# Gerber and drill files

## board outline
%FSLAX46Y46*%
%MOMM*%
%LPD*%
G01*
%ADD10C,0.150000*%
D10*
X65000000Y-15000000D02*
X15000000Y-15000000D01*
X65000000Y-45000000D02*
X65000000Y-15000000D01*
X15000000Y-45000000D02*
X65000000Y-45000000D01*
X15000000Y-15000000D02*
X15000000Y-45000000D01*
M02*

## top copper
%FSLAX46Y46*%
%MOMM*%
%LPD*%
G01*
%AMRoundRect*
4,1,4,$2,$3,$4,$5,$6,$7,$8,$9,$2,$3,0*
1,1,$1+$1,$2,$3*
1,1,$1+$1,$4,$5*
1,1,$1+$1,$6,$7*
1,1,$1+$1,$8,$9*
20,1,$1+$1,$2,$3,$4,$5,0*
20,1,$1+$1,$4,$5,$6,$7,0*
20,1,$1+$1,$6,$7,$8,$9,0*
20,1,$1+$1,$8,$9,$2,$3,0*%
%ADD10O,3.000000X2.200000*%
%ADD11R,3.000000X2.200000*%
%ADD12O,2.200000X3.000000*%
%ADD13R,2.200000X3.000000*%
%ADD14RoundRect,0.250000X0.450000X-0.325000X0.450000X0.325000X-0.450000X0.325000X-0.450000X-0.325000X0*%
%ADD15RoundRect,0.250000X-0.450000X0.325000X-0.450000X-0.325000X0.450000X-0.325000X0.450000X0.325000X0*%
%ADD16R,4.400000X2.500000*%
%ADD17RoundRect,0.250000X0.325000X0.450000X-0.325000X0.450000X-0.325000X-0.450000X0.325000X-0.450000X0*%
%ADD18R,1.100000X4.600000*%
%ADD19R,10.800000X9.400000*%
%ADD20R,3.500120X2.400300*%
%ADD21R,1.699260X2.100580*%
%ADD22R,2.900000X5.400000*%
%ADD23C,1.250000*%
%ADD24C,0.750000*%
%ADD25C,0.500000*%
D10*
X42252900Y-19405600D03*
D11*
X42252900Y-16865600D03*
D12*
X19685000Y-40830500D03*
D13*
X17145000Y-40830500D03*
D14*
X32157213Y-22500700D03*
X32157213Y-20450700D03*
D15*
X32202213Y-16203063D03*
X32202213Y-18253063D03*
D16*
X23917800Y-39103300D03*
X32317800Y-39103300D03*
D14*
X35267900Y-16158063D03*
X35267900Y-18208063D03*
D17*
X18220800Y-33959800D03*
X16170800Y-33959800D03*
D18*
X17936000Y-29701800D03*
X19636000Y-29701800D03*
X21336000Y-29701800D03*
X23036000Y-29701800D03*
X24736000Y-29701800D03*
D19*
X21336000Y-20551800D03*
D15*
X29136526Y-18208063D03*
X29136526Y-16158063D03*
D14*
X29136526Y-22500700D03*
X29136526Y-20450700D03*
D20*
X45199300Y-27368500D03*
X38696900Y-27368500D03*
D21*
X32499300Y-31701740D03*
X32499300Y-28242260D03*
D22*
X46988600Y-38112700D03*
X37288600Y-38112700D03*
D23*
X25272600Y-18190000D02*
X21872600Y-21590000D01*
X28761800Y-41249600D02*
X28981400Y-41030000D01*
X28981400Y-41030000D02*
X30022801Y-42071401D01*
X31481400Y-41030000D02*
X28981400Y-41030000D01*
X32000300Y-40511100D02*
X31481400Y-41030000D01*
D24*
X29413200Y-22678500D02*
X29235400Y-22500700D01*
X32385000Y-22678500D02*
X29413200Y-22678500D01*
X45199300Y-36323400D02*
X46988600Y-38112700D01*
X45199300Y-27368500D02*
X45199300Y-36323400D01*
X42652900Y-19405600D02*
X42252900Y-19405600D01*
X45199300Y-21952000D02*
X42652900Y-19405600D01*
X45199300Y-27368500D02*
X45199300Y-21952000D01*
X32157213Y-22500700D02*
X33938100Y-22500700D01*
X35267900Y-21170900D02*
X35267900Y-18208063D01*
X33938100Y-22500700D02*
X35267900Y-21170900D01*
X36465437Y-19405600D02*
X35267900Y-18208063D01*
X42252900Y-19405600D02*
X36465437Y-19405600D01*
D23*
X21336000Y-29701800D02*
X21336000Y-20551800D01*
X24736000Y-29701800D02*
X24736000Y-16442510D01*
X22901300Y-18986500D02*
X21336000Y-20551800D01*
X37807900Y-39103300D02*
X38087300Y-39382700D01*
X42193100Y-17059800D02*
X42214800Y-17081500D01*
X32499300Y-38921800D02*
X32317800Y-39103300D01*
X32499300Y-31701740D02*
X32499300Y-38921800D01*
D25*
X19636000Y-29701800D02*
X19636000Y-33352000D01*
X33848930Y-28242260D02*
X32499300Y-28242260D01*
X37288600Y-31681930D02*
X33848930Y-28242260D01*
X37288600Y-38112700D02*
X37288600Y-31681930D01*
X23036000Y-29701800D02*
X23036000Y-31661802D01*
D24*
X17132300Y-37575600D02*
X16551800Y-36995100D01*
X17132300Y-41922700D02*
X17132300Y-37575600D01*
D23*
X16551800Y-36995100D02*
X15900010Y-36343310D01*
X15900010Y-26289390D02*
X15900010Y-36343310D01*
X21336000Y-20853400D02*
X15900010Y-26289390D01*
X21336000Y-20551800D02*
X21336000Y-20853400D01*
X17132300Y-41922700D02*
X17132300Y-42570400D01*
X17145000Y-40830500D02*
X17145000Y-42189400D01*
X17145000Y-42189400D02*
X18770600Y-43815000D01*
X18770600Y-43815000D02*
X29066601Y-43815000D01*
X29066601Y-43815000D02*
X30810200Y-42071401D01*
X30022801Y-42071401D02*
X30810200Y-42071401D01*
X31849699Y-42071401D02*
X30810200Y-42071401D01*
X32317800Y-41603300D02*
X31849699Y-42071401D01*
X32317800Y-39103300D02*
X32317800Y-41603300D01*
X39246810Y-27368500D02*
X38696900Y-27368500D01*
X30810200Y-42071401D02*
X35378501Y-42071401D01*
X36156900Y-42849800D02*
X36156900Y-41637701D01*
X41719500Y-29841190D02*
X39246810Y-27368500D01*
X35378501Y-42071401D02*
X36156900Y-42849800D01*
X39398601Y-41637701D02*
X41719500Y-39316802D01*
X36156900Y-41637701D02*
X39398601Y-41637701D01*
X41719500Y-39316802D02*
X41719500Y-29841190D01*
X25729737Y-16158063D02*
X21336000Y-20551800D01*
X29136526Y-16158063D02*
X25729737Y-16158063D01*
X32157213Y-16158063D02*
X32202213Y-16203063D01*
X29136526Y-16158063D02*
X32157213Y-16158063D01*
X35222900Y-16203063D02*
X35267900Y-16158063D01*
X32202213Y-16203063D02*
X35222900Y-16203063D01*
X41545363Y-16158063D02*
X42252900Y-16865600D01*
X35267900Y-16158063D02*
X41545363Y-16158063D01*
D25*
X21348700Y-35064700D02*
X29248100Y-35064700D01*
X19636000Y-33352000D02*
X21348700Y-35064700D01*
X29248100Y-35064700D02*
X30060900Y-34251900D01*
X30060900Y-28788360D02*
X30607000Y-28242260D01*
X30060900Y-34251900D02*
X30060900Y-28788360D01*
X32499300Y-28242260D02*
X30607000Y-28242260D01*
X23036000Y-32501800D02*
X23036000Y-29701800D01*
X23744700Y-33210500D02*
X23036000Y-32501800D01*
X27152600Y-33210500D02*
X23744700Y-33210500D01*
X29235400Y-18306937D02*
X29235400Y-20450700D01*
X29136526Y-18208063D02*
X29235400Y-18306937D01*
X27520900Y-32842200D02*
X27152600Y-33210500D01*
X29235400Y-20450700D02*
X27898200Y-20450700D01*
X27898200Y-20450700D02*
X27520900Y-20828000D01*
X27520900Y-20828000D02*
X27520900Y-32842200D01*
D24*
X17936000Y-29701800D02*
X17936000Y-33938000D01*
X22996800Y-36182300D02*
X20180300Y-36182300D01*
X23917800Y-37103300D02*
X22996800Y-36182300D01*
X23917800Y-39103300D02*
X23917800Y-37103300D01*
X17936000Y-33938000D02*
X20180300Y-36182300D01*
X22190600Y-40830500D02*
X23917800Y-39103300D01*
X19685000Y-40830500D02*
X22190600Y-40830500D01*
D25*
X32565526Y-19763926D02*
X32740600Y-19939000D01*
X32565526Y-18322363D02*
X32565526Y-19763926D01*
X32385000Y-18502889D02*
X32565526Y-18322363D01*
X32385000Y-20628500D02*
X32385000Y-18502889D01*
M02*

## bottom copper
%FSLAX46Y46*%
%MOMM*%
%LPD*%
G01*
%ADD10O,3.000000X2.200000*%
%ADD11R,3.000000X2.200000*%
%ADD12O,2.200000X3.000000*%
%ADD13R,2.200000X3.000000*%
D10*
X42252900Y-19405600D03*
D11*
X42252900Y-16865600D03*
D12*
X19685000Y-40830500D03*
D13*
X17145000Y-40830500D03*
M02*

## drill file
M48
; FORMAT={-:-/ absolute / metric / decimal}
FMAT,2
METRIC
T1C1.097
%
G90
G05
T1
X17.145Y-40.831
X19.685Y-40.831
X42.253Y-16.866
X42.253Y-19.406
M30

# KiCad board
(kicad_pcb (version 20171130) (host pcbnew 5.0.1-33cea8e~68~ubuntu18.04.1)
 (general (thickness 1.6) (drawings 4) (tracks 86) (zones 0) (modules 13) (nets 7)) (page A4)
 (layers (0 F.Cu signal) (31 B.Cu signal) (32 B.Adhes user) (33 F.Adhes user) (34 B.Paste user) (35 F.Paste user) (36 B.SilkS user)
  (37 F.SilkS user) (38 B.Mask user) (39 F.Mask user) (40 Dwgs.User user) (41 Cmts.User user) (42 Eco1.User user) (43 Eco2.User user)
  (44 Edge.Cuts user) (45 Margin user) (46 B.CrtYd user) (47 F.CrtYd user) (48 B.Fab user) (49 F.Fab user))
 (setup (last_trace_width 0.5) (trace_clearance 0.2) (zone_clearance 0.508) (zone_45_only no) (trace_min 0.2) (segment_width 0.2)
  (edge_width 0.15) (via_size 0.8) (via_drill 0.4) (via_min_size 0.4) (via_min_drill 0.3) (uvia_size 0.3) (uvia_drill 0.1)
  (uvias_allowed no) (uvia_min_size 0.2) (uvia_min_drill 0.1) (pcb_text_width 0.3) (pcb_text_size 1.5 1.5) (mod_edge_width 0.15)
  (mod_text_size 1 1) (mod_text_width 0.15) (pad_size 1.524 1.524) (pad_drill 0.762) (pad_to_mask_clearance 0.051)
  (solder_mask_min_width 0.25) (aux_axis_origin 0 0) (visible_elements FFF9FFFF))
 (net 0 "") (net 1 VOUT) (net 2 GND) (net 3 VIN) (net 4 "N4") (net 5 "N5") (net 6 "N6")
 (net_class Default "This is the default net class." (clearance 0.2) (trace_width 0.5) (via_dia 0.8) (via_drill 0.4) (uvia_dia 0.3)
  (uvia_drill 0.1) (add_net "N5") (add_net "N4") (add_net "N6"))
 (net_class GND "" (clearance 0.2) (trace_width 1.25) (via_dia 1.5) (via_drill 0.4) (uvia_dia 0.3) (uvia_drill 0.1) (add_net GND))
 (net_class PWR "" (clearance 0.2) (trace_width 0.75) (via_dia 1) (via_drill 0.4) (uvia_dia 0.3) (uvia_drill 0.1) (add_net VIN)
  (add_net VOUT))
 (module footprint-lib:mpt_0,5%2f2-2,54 (layer F.Cu) (at 42.2529 18.1356 90)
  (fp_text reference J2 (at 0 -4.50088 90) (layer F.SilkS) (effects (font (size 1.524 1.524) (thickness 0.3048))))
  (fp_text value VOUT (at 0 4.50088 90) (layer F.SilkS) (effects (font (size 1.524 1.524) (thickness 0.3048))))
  (pad 2 thru_hole oval (at -1.27 0 90) (size 2.2 3) (drill 1.09728) (layers *.Cu *.Mask) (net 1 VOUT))
  (pad 1 thru_hole rect (at 1.27 0 90) (size 2.2 3) (drill 1.09728) (layers *.Cu *.Mask) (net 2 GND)))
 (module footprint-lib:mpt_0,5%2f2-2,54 (layer F.Cu) (at 18.415 40.8305 180)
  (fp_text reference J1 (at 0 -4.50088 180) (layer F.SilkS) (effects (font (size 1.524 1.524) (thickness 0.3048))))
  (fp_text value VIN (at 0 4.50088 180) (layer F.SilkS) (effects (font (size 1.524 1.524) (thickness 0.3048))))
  (pad 2 thru_hole oval (at -1.27 0 180) (size 2.2 3) (drill 1.09728) (layers *.Cu *.Mask) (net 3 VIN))
  (pad 1 thru_hole rect (at 1.27 0 180) (size 2.2 3) (drill 1.09728) (layers *.Cu *.Mask) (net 2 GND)))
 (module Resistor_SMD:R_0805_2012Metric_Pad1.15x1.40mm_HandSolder (layer F.Cu) (at 32.157213 21.4757 90)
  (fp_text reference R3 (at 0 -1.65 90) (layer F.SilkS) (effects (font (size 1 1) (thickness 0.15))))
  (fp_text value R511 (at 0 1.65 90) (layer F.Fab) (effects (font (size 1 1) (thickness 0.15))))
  (pad 1 smd roundrect (at -1.025 0 90) (size 1.15 1.4) (layers F.Cu F.Paste F.Mask) (roundrect_rratio 0.217391) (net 1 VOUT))
  (pad 2 smd roundrect (at 1.025 0 90) (size 1.15 1.4) (layers F.Cu F.Paste F.Mask) (roundrect_rratio 0.217391) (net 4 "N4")))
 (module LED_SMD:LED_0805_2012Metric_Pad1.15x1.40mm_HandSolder (layer F.Cu) (at 32.202213 17.228063 270)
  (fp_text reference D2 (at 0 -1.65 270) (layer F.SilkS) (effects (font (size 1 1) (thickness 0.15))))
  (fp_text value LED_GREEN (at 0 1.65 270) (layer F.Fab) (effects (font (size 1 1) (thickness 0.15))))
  (pad 1 smd roundrect (at -1.025 0 270) (size 1.15 1.4) (layers F.Cu F.Paste F.Mask) (roundrect_rratio 0.217391) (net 2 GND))
  (pad 2 smd roundrect (at 1.025 0 270) (size 1.15 1.4) (layers F.Cu F.Paste F.Mask) (roundrect_rratio 0.217391) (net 4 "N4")))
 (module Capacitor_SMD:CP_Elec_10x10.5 (layer F.Cu) (at 28.1178 39.1033)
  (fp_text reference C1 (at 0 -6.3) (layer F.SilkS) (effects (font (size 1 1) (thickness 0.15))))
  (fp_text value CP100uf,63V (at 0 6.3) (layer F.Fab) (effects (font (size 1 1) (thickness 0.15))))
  (pad 1 smd rect (at -4.2 0) (size 4.4 2.5) (layers F.Cu F.Paste F.Mask) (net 3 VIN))
  (pad 2 smd rect (at 4.2 0) (size 4.4 2.5) (layers F.Cu F.Paste F.Mask) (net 2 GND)))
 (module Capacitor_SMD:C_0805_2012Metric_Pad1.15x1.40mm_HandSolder (layer F.Cu) (at 35.2679 17.183063 90)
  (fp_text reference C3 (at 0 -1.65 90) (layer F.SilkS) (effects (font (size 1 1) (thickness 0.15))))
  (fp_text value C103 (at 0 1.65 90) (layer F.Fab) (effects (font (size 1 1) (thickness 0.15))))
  (pad 2 smd roundrect (at 1.025 0 90) (size 1.15 1.4) (layers F.Cu F.Paste F.Mask) (roundrect_rratio 0.217391) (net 2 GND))
  (pad 1 smd roundrect (at -1.025 0 90) (size 1.15 1.4) (layers F.Cu F.Paste F.Mask) (roundrect_rratio 0.217391) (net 1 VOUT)))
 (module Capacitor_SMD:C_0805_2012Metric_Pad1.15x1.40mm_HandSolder (layer F.Cu) (at 17.1958 33.9598 180)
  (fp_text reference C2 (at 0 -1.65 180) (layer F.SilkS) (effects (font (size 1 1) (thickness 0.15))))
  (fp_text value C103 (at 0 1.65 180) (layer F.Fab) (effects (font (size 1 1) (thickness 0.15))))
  (pad 1 smd roundrect (at -1.025 0 180) (size 1.15 1.4) (layers F.Cu F.Paste F.Mask) (roundrect_rratio 0.217391) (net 3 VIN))
  (pad 2 smd roundrect (at 1.025 0 180) (size 1.15 1.4) (layers F.Cu F.Paste F.Mask) (roundrect_rratio 0.217391) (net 2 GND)))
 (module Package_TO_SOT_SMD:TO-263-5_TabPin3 (layer F.Cu) (at 21.336 23.9268 90)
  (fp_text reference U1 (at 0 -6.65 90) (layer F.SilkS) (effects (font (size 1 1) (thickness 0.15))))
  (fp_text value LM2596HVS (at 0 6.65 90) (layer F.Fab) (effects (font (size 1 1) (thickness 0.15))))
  (pad 1 smd rect (at -5.775 -3.4 90) (size 4.6 1.1) (layers F.Cu F.Paste F.Mask) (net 3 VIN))
  (pad 2 smd rect (at -5.775 -1.7 90) (size 4.6 1.1) (layers F.Cu F.Paste F.Mask) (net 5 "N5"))
  (pad 3 smd rect (at -5.775 0 90) (size 4.6 1.1) (layers F.Cu F.Paste F.Mask) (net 2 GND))
  (pad 4 smd rect (at -5.775 1.7 90) (size 4.6 1.1) (layers F.Cu F.Paste F.Mask) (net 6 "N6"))
  (pad 5 smd rect (at -5.775 3.4 90) (size 4.6 1.1) (layers F.Cu F.Paste F.Mask) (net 2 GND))
  (pad 3 smd rect (at 3.375 0 90) (size 9.4 10.8) (layers F.Cu F.Mask) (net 2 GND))
  (pad "" smd rect (at 5.8 2.775 90) (size 4.55 5.25) (layers F.Paste))
  (pad "" smd rect (at 0.95 -2.775 90) (size 4.55 5.25) (layers F.Paste))
  (pad "" smd rect (at 5.8 -2.775 90) (size 4.55 5.25) (layers F.Paste))
  (pad "" smd rect (at 0.95 2.775 90) (size 4.55 5.25) (layers F.Paste)))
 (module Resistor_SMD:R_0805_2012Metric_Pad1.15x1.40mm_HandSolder (layer F.Cu) (at 29.136526 17.183063 270)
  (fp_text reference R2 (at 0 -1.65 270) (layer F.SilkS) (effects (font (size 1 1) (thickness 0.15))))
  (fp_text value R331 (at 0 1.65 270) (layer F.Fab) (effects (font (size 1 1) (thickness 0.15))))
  (pad 2 smd roundrect (at 1.025 0 270) (size 1.15 1.4) (layers F.Cu F.Paste F.Mask) (roundrect_rratio 0.217391) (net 6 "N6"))
  (pad 1 smd roundrect (at -1.025 0 270) (size 1.15 1.4) (layers F.Cu F.Paste F.Mask) (roundrect_rratio 0.217391) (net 2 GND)))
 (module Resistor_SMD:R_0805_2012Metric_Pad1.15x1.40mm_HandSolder (layer F.Cu) (at 29.136526 21.4757 90)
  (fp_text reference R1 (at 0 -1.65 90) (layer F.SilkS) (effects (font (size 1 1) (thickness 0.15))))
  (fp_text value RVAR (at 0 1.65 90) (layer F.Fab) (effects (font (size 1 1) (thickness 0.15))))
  (pad 1 smd roundrect (at -1.025 0 90) (size 1.15 1.4) (layers F.Cu F.Paste F.Mask) (roundrect_rratio 0.217391) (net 1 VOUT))
  (pad 2 smd roundrect (at 1.025 0 90) (size 1.15 1.4) (layers F.Cu F.Paste F.Mask) (roundrect_rratio 0.217391) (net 6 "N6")))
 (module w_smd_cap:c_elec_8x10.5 (layer F.Cu) (at 41.9481 27.3685)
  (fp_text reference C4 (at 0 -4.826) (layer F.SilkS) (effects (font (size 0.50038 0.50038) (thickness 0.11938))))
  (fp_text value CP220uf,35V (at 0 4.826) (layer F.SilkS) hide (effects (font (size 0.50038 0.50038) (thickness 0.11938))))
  (pad 1 smd rect (at 3.2512 0) (size 3.50012 2.4003) (layers F.Cu F.Paste F.Mask) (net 1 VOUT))
  (pad 2 smd rect (at -3.2512 0) (size 3.50012 2.4003) (layers F.Cu F.Paste F.Mask) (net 2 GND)))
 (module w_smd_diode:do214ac (layer F.Cu) (at 32.4993 29.972 270)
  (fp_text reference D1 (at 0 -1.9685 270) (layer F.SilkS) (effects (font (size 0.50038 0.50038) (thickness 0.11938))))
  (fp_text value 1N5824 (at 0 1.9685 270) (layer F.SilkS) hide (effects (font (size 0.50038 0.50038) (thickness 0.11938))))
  (pad 2 smd rect (at 1.72974 0 270) (size 2.10058 1.69926) (layers F.Cu F.Paste F.Mask) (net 2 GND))
  (pad 1 smd rect (at -1.72974 0 270) (size 2.10058 1.69926) (layers F.Cu F.Paste F.Mask) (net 5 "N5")))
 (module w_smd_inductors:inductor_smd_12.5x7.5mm (layer F.Cu) (at 42.1386 38.1127 90)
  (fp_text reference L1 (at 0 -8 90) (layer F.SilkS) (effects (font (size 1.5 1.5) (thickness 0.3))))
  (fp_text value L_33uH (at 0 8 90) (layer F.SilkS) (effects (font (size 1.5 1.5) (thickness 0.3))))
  (pad 2 smd rect (at 0 4.85 90) (size 5.4 2.9) (layers F.Cu F.Paste F.Mask) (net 1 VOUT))
  (pad 1 smd rect (at 0 -4.85 90) (size 5.4 2.9) (layers F.Cu F.Paste F.Mask) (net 5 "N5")))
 (gr_line (start 65 15) (end 15 15) (layer Edge.Cuts) (width 0.15))
 (gr_line (start 65 45) (end 65 15) (layer Edge.Cuts) (width 0.15))
 (gr_line (start 15 45) (end 65 45) (layer Edge.Cuts) (width 0.15))
 (gr_line (start 15 15) (end 15 45) (layer Edge.Cuts) (width 0.15))
 (segment (start 25.2726 18.19) (end 21.8726 21.59) (width 1.25) (layer F.Cu) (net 2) (status 30))
 (segment (start 28.7618 41.2496) (end 28.9814 41.03) (width 1.25) (layer F.Cu) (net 2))
 (segment (start 28.9814 41.03) (end 30.022801 42.071401) (width 1.25) (layer F.Cu) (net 2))
 (segment (start 31.4814 41.03) (end 28.9814 41.03) (width 1.25) (layer F.Cu) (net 2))
 (segment (start 32.0003 40.5111) (end 31.4814 41.03) (width 1.25) (layer F.Cu) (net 2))
 (segment (start 29.4132 22.6785) (end 29.2354 22.5007) (width 0.75) (layer F.Cu) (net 1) (status 30))
 (segment (start 32.385 22.6785) (end 29.4132 22.6785) (width 0.75) (layer F.Cu) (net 1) (status 30))
 (segment (start 45.1993 36.3234) (end 46.9886 38.1127) (width 0.75) (layer F.Cu) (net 1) (status 20))
 (segment (start 45.1993 27.3685) (end 45.1993 36.3234) (width 0.75) (layer F.Cu) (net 1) (status 10))
 (segment (start 42.6529 19.4056) (end 42.2529 19.4056) (width 0.75) (layer F.Cu) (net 1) (status 30))
 (segment (start 45.1993 21.952) (end 42.6529 19.4056) (width 0.75) (layer F.Cu) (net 1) (status 20))
 (segment (start 45.1993 27.3685) (end 45.1993 21.952) (width 0.75) (layer F.Cu) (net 1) (status 10))
 (segment (start 32.157213 22.5007) (end 33.9381 22.5007) (width 0.75) (layer F.Cu) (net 1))
 (segment (start 35.2679 21.1709) (end 35.2679 18.208063) (width 0.75) (layer F.Cu) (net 1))
 (segment (start 33.9381 22.5007) (end 35.2679 21.1709) (width 0.75) (layer F.Cu) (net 1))
 (segment (start 36.465437 19.4056) (end 35.2679 18.208063) (width 0.75) (layer F.Cu) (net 1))
 (segment (start 42.2529 19.4056) (end 36.465437 19.4056) (width 0.75) (layer F.Cu) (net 1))
 (segment (start 21.336 29.7018) (end 21.336 20.5518) (width 1.25) (layer F.Cu) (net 2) (status 30))
 (segment (start 24.736 29.7018) (end 24.736 16.44251) (width 1.25) (layer F.Cu) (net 2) (status 30))
 (segment (start 22.9013 18.9865) (end 21.336 20.5518) (width 1.25) (layer F.Cu) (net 2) (status 30))
 (segment (start 37.8079 39.1033) (end 38.0873 39.3827) (width 1.25) (layer F.Cu) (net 5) (status 30))
 (segment (start 42.1931 17.0598) (end 42.2148 17.0815) (width 1.25) (layer F.Cu) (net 2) (status 30))
 (segment (start 32.4993 38.9218) (end 32.3178 39.1033) (width 1.25) (layer F.Cu) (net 2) (status 30))
 (segment (start 32.4993 31.70174) (end 32.4993 38.9218) (width 1.25) (layer F.Cu) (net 2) (status 30))
 (segment (start 19.636 29.7018) (end 19.636 33.352) (width 0.5) (layer F.Cu) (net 5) (status 10))
 (segment (start 33.84893 28.24226) (end 32.4993 28.24226) (width 0.5) (layer F.Cu) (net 5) (status 20))
 (segment (start 37.2886 31.68193) (end 33.84893 28.24226) (width 0.5) (layer F.Cu) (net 5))
 (segment (start 37.2886 38.1127) (end 37.2886 31.68193) (width 0.5) (layer F.Cu) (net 5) (status 10))
 (segment (start 23.036 29.7018) (end 23.036 31.661802) (width 0.5) (layer F.Cu) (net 6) (status 30))
 (segment (start 17.1323 37.5756) (end 16.5518 36.9951) (width 0.75) (layer F.Cu) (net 2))
 (segment (start 17.1323 41.9227) (end 17.1323 37.5756) (width 0.75) (layer F.Cu) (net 2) (status 10))
 (segment (start 16.5518 36.9951) (end 15.90001 36.34331) (width 1.25) (layer F.Cu) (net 2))
 (segment (start 15.90001 26.28939) (end 15.90001 36.34331) (width 1.25) (layer F.Cu) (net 2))
 (segment (start 21.336 20.8534) (end 15.90001 26.28939) (width 1.25) (layer F.Cu) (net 2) (status 10))
 (segment (start 21.336 20.5518) (end 21.336 20.8534) (width 1.25) (layer F.Cu) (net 2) (status 30))
 (segment (start 17.1323 41.9227) (end 17.1323 42.5704) (width 1.25) (layer F.Cu) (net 2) (status 10))
 (segment (start 17.145 40.8305) (end 17.145 42.1894) (width 1.25) (layer F.Cu) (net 2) (status 30))
 (segment (start 17.145 42.1894) (end 18.7706 43.815) (width 1.25) (layer F.Cu) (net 2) (status 10))
 (segment (start 18.7706 43.815) (end 29.066601 43.815) (width 1.25) (layer F.Cu) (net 2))
 (segment (start 29.066601 43.815) (end 30.8102 42.071401) (width 1.25) (layer F.Cu) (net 2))
 (segment (start 30.022801 42.071401) (end 30.8102 42.071401) (width 1.25) (layer F.Cu) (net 2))
 (segment (start 31.849699 42.071401) (end 30.8102 42.071401) (width 1.25) (layer F.Cu) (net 2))
 (segment (start 32.3178 41.6033) (end 31.849699 42.071401) (width 1.25) (layer F.Cu) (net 2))
 (segment (start 32.3178 39.1033) (end 32.3178 41.6033) (width 1.25) (layer F.Cu) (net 2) (status 10))
 (segment (start 39.24681 27.3685) (end 38.6969 27.3685) (width 1.25) (layer F.Cu) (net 2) (status 30))
 (segment (start 30.8102 42.071401) (end 35.378501 42.071401) (width 1.25) (layer F.Cu) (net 2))
 (segment (start 36.1569 42.8498) (end 36.1569 41.637701) (width 1.25) (layer F.Cu) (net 2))
 (segment (start 41.7195 29.84119) (end 39.24681 27.3685) (width 1.25) (layer F.Cu) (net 2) (status 20))
 (segment (start 35.378501 42.071401) (end 36.1569 42.8498) (width 1.25) (layer F.Cu) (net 2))
 (segment (start 39.398601 41.637701) (end 41.7195 39.316802) (width 1.25) (layer F.Cu) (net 2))
 (segment (start 36.1569 41.637701) (end 39.398601 41.637701) (width 1.25) (layer F.Cu) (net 2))
 (segment (start 41.7195 39.316802) (end 41.7195 29.84119) (width 1.25) (layer F.Cu) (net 2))
 (segment (start 25.729737 16.158063) (end 21.336 20.5518) (width 1.25) (layer F.Cu) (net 2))
 (segment (start 29.136526 16.158063) (end 25.729737 16.158063) (width 1.25) (layer F.Cu) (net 2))
 (segment (start 32.157213 16.158063) (end 32.202213 16.203063) (width 1.25) (layer F.Cu) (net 2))
 (segment (start 29.136526 16.158063) (end 32.157213 16.158063) (width 1.25) (layer F.Cu) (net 2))
 (segment (start 35.2229 16.203063) (end 35.2679 16.158063) (width 1.25) (layer F.Cu) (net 2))
 (segment (start 32.202213 16.203063) (end 35.2229 16.203063) (width 1.25) (layer F.Cu) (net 2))
 (segment (start 41.545363 16.158063) (end 42.2529 16.8656) (width 1.25) (layer F.Cu) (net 2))
 (segment (start 35.2679 16.158063) (end 41.545363 16.158063) (width 1.25) (layer F.Cu) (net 2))
 (segment (start 21.3487 35.0647) (end 29.2481 35.0647) (width 0.5) (layer F.Cu) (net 5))
 (segment (start 19.636 33.352) (end 21.3487 35.0647) (width 0.5) (layer F.Cu) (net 5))
 (segment (start 29.2481 35.0647) (end 30.0609 34.2519) (width 0.5) (layer F.Cu) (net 5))
 (segment (start 30.0609 28.78836) (end 30.607 28.24226) (width 0.5) (layer F.Cu) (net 5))
 (segment (start 30.0609 34.2519) (end 30.0609 28.78836) (width 0.5) (layer F.Cu) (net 5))
 (segment (start 32.4993 28.24226) (end 30.607 28.24226) (width 0.5) (layer F.Cu) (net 5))
 (segment (start 23.036 32.5018) (end 23.036 29.7018) (width 0.5) (layer F.Cu) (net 6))
 (segment (start 23.7447 33.2105) (end 23.036 32.5018) (width 0.5) (layer F.Cu) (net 6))
 (segment (start 27.1526 33.2105) (end 23.7447 33.2105) (width 0.5) (layer F.Cu) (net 6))
 (segment (start 29.2354 18.306937) (end 29.2354 20.4507) (width 0.5) (layer F.Cu) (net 6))
 (segment (start 29.136526 18.208063) (end 29.2354 18.306937) (width 0.5) (layer F.Cu) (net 6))
 (segment (start 27.5209 32.8422) (end 27.1526 33.2105) (width 0.5) (layer F.Cu) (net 6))
 (segment (start 29.2354 20.4507) (end 27.8982 20.4507) (width 0.5) (layer F.Cu) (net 6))
 (segment (start 27.8982 20.4507) (end 27.5209 20.828) (width 0.5) (layer F.Cu) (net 6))
 (segment (start 27.5209 20.828) (end 27.5209 32.8422) (width 0.5) (layer F.Cu) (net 6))
 (segment (start 17.936 29.7018) (end 17.936 33.938) (width 0.75) (layer F.Cu) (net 3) (status 30))
 (segment (start 22.9968 36.1823) (end 20.1803 36.1823) (width 0.75) (layer F.Cu) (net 3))
 (segment (start 23.9178 37.1033) (end 22.9968 36.1823) (width 0.75) (layer F.Cu) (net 3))
 (segment (start 23.9178 39.1033) (end 23.9178 37.1033) (width 0.75) (layer F.Cu) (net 3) (status 10))
 (segment (start 17.936 33.938) (end 20.1803 36.1823) (width 0.75) (layer F.Cu) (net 3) (status 10))
 (segment (start 22.1906 40.8305) (end 23.9178 39.1033) (width 0.75) (layer F.Cu) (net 3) (status 20))
 (segment (start 19.685 40.8305) (end 22.1906 40.8305) (width 0.75) (layer F.Cu) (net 3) (status 10))
 (segment (start 32.565526 19.763926) (end 32.7406 19.939) (width 0.5) (layer F.Cu) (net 4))
 (segment (start 32.565526 18.322363) (end 32.565526 19.763926) (width 0.5) (layer F.Cu) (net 4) (status 10))
 (segment (start 32.385 18.502889) (end 32.565526 18.322363) (width 0.5) (layer F.Cu) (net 4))
 (segment (start 32.385 20.6285) (end 32.385 18.502889) (width 0.5) (layer F.Cu) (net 4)))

